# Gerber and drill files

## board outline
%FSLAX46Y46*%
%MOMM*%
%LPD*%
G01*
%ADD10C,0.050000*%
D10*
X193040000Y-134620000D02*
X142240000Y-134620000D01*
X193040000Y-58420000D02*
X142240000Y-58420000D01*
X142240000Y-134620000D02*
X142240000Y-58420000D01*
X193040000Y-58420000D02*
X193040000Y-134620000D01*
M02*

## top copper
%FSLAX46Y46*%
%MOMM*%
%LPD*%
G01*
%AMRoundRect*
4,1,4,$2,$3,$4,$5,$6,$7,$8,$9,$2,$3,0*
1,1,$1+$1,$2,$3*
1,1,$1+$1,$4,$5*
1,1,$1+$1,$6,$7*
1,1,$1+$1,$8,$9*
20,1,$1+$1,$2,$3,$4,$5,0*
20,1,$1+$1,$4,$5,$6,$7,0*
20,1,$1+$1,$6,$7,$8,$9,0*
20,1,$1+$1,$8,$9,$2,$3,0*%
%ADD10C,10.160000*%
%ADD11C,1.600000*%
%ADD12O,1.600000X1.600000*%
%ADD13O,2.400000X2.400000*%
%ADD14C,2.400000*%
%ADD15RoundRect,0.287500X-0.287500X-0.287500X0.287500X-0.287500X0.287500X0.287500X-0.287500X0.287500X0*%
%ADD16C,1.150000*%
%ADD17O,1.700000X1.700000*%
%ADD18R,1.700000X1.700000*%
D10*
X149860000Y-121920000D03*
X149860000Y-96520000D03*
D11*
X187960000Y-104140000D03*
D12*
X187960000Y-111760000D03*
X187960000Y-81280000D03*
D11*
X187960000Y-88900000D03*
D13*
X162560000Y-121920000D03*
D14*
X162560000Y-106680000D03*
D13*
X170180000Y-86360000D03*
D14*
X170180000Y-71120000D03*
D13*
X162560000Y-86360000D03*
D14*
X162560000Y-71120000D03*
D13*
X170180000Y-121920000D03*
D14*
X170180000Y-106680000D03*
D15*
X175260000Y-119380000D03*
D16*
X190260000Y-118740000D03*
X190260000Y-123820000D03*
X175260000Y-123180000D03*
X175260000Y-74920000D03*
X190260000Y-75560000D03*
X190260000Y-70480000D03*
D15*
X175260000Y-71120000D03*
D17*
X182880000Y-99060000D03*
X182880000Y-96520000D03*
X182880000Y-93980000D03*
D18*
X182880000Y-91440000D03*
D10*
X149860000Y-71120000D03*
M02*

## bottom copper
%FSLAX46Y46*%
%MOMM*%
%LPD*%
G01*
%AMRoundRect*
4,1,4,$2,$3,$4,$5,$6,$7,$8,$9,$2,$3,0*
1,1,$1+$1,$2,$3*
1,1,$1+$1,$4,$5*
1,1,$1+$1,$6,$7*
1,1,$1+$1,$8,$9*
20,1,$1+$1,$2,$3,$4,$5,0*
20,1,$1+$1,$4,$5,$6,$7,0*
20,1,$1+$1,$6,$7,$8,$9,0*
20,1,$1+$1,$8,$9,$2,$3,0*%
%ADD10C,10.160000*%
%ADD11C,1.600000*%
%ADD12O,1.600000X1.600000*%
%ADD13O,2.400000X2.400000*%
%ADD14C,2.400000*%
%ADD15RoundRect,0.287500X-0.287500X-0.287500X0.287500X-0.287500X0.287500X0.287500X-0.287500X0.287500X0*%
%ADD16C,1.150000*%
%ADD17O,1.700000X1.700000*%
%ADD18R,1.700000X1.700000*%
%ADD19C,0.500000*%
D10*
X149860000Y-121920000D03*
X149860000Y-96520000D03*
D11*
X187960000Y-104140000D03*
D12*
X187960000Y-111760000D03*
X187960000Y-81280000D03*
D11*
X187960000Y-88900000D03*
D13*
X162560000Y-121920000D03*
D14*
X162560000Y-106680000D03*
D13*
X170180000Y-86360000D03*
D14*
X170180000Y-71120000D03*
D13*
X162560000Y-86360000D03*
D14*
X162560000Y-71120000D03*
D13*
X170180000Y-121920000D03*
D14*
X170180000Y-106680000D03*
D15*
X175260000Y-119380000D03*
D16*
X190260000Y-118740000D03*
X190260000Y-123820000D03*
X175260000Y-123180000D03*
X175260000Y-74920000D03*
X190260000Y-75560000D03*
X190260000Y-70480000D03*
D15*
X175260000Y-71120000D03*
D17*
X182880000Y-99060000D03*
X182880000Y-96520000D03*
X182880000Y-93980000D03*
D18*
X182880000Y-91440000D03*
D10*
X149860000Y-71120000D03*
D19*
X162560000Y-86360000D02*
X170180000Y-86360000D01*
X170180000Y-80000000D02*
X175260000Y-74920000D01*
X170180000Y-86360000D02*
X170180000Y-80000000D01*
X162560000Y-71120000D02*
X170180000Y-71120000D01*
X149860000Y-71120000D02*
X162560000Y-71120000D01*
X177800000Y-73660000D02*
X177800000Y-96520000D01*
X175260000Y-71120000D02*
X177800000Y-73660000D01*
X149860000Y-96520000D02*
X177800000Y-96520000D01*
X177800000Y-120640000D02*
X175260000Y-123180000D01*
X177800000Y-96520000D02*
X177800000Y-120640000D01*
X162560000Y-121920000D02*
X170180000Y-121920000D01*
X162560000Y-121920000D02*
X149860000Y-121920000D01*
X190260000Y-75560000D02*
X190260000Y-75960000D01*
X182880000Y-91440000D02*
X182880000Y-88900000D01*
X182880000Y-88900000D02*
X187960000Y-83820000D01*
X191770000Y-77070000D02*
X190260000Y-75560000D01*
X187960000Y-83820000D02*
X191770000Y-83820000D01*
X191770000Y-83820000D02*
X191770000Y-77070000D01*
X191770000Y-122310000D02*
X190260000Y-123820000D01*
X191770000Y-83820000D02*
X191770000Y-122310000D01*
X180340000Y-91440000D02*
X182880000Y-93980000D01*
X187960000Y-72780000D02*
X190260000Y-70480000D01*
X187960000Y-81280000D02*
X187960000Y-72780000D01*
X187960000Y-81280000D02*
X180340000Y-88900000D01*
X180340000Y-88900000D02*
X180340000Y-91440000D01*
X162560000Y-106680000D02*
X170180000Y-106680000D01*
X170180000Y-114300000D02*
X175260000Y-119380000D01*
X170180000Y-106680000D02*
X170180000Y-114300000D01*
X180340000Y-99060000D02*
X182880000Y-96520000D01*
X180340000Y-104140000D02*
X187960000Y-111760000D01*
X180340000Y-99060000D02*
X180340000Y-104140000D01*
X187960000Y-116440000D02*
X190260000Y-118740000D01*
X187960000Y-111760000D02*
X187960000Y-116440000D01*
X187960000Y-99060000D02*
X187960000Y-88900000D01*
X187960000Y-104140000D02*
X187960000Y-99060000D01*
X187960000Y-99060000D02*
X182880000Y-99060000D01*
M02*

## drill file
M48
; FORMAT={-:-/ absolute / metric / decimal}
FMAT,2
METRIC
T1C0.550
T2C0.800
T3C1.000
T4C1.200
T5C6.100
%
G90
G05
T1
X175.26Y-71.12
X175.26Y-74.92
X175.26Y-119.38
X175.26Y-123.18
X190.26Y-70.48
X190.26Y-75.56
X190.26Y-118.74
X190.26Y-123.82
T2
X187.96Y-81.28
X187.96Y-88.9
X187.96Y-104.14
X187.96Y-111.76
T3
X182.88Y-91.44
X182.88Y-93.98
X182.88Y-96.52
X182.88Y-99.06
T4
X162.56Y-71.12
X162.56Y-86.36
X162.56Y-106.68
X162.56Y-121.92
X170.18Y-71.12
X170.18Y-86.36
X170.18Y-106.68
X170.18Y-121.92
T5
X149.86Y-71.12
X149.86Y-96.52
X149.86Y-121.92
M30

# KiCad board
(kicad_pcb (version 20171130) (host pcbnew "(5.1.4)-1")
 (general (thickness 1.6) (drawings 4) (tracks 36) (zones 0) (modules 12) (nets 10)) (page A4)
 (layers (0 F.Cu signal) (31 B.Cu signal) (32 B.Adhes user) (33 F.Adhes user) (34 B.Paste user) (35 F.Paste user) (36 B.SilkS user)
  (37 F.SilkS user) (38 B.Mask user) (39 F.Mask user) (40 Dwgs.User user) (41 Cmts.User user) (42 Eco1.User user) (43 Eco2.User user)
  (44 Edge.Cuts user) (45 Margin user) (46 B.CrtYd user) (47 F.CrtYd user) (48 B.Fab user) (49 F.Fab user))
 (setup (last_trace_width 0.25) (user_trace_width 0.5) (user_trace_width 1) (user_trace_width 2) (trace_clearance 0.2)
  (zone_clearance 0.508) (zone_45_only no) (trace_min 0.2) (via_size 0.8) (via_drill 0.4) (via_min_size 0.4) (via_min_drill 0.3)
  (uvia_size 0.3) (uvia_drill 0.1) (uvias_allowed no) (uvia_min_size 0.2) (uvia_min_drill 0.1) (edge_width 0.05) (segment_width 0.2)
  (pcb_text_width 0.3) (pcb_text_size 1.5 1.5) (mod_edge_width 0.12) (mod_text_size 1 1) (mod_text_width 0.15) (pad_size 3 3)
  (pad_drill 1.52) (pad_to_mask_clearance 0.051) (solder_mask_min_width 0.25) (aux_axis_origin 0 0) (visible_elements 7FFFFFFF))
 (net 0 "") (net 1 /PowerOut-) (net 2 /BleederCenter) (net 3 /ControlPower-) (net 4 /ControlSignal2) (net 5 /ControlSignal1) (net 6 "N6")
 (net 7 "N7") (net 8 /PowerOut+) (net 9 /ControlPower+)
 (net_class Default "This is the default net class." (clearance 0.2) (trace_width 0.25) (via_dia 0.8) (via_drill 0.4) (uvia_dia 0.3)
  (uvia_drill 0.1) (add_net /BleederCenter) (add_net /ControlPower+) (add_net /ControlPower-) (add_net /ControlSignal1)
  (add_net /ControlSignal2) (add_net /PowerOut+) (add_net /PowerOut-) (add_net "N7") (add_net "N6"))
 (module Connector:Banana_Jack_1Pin (layer F.Cu) (at 149.86 121.92)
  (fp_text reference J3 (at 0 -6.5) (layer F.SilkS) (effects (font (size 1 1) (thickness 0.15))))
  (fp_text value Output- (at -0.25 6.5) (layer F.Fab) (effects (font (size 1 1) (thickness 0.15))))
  (pad 1 thru_hole circle (at 0 0) (size 10.16 10.16) (drill 6.1) (layers *.Cu *.Mask) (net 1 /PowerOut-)))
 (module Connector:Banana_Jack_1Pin (layer F.Cu) (at 149.86 96.52)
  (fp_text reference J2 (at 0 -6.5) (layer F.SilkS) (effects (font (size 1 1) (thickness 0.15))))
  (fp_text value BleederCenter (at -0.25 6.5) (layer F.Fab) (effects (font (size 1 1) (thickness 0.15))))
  (pad 1 thru_hole circle (at 0 0) (size 10.16 10.16) (drill 6.1) (layers *.Cu *.Mask) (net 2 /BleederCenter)))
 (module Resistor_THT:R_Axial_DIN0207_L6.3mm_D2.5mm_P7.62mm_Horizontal (layer F.Cu) (at 187.96 104.14 270)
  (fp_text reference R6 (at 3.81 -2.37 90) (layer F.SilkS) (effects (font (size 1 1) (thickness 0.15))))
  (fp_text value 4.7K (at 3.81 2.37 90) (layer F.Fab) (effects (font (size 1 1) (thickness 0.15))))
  (pad 1 thru_hole circle (at 0 0 270) (size 1.6 1.6) (drill 0.8) (layers *.Cu *.Mask) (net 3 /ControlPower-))
  (pad 2 thru_hole oval (at 7.62 0 270) (size 1.6 1.6) (drill 0.8) (layers *.Cu *.Mask) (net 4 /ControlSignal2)))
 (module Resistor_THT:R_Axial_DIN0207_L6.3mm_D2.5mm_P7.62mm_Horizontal (layer F.Cu) (at 187.96 88.9 90)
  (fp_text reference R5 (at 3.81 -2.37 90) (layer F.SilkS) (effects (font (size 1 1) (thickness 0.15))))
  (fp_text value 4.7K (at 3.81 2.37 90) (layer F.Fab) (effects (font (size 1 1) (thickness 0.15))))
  (pad 2 thru_hole oval (at 7.62 0 90) (size 1.6 1.6) (drill 0.8) (layers *.Cu *.Mask) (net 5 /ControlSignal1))
  (pad 1 thru_hole circle (at 0 0 90) (size 1.6 1.6) (drill 0.8) (layers *.Cu *.Mask) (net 3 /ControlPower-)))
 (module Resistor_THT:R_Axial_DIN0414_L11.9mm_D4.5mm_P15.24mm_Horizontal (layer F.Cu) (at 162.56 106.68 270)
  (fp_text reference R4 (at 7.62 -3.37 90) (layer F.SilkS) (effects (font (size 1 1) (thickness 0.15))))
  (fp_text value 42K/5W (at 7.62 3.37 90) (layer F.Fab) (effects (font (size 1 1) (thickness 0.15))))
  (pad 2 thru_hole oval (at 15.24 0 270) (size 2.4 2.4) (drill 1.2) (layers *.Cu *.Mask) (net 1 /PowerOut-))
  (pad 1 thru_hole circle (at 0 0 270) (size 2.4 2.4) (drill 1.2) (layers *.Cu *.Mask) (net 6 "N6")))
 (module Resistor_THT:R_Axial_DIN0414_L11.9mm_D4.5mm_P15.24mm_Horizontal (layer F.Cu) (at 170.18 71.12 270)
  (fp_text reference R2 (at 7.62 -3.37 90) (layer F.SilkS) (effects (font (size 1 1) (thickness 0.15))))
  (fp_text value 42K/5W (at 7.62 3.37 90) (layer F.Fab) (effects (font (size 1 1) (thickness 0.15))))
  (pad 2 thru_hole oval (at 15.24 0 270) (size 2.4 2.4) (drill 1.2) (layers *.Cu *.Mask) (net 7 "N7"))
  (pad 1 thru_hole circle (at 0 0 270) (size 2.4 2.4) (drill 1.2) (layers *.Cu *.Mask) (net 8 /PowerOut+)))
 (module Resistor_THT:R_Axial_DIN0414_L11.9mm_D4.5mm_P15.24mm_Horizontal (layer F.Cu) (at 162.56 71.12 270)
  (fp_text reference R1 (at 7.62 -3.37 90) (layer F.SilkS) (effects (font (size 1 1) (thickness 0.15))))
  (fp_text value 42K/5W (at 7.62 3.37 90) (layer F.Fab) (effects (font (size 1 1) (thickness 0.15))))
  (pad 2 thru_hole oval (at 15.24 0 270) (size 2.4 2.4) (drill 1.2) (layers *.Cu *.Mask) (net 7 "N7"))
  (pad 1 thru_hole circle (at 0 0 270) (size 2.4 2.4) (drill 1.2) (layers *.Cu *.Mask) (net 8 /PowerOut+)))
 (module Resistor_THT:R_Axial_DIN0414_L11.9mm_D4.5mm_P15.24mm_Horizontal (layer F.Cu) (at 170.18 106.68 270)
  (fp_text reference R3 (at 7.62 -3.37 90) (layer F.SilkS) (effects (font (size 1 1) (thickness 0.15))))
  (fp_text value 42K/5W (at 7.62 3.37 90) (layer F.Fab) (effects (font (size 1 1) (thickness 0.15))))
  (pad 2 thru_hole oval (at 15.24 0 270) (size 2.4 2.4) (drill 1.2) (layers *.Cu *.Mask) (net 1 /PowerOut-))
  (pad 1 thru_hole circle (at 0 0 270) (size 2.4 2.4) (drill 1.2) (layers *.Cu *.Mask) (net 6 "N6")))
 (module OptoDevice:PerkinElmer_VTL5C (layer F.Cu) (at 175.26 119.38)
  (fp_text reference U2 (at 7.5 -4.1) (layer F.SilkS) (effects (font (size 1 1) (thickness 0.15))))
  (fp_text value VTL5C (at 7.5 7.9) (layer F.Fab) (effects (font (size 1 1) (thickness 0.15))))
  (pad 1 thru_hole roundrect (at 0 0) (size 1.15 1.15) (drill 0.55) (layers *.Cu *.Mask) (roundrect_rratio 0.25) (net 6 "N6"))
  (pad 3 thru_hole circle (at 15 -0.64) (size 1.15 1.15) (drill 0.55) (layers *.Cu *.Mask) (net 4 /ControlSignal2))
  (pad 4 thru_hole circle (at 15 4.44) (size 1.15 1.15) (drill 0.55) (layers *.Cu *.Mask) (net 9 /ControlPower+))
  (pad 2 thru_hole circle (at 0 3.8) (size 1.15 1.15) (drill 0.55) (layers *.Cu *.Mask) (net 2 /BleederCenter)))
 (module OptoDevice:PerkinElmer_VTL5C (layer F.Cu) (at 175.26 71.12)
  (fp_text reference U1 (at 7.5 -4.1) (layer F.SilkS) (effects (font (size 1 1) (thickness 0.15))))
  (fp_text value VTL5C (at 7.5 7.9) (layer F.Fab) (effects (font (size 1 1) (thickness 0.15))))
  (pad 2 thru_hole circle (at 0 3.8) (size 1.15 1.15) (drill 0.55) (layers *.Cu *.Mask) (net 7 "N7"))
  (pad 4 thru_hole circle (at 15 4.44) (size 1.15 1.15) (drill 0.55) (layers *.Cu *.Mask) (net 9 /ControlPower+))
  (pad 3 thru_hole circle (at 15 -0.64) (size 1.15 1.15) (drill 0.55) (layers *.Cu *.Mask) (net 5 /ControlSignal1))
  (pad 1 thru_hole roundrect (at 0 0) (size 1.15 1.15) (drill 0.55) (layers *.Cu *.Mask) (roundrect_rratio 0.25) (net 2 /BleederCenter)))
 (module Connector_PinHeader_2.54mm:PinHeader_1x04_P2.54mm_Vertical (layer F.Cu) (at 182.88 91.44)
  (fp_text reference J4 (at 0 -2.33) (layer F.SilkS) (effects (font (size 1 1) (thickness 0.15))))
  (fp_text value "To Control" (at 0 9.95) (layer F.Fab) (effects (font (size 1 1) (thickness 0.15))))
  (pad 4 thru_hole oval (at 0 7.62) (size 1.7 1.7) (drill 1) (layers *.Cu *.Mask) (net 3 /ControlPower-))
  (pad 3 thru_hole oval (at 0 5.08) (size 1.7 1.7) (drill 1) (layers *.Cu *.Mask) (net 4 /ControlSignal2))
  (pad 2 thru_hole oval (at 0 2.54) (size 1.7 1.7) (drill 1) (layers *.Cu *.Mask) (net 5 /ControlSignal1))
  (pad 1 thru_hole rect (at 0 0) (size 1.7 1.7) (drill 1) (layers *.Cu *.Mask) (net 9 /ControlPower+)))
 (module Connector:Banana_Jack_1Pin (layer F.Cu) (at 149.86 71.12)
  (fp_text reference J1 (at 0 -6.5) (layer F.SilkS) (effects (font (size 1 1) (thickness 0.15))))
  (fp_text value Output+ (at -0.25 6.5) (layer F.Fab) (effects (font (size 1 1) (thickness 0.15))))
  (pad 1 thru_hole circle (at 0 0) (size 10.16 10.16) (drill 6.1) (layers *.Cu *.Mask) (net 8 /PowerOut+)))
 (gr_line (start 193.04 134.62) (end 142.24 134.62) (layer Edge.Cuts) (width 0.05))
 (gr_line (start 193.04 58.42) (end 142.24 58.42) (layer Edge.Cuts) (width 0.05))
 (gr_line (start 142.24 134.62) (end 142.24 58.42) (layer Edge.Cuts) (width 0.05))
 (gr_line (start 193.04 58.42) (end 193.04 134.62) (layer Edge.Cuts) (width 0.05))
 (segment (start 162.56 86.36) (end 170.18 86.36) (width 0.5) (layer B.Cu) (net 7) (status 30))
 (segment (start 170.18 80) (end 175.26 74.92) (width 0.5) (layer B.Cu) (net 7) (status 20))
 (segment (start 170.18 86.36) (end 170.18 80) (width 0.5) (layer B.Cu) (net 7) (status 10))
 (segment (start 162.56 71.12) (end 170.18 71.12) (width 0.5) (layer B.Cu) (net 8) (status 30))
 (segment (start 149.86 71.12) (end 162.56 71.12) (width 0.5) (layer B.Cu) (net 8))
 (segment (start 177.8 73.66) (end 177.8 96.52) (width 0.5) (layer B.Cu) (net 2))
 (segment (start 175.26 71.12) (end 177.8 73.66) (width 0.5) (layer B.Cu) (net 2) (status 10))
 (segment (start 149.86 96.52) (end 177.8 96.52) (width 0.5) (layer B.Cu) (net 2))
 (segment (start 177.8 120.64) (end 175.26 123.18) (width 0.5) (layer B.Cu) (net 2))
 (segment (start 177.8 96.52) (end 177.8 120.64) (width 0.5) (layer B.Cu) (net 2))
 (segment (start 162.56 121.92) (end 170.18 121.92) (width 0.5) (layer B.Cu) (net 1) (status 30))
 (segment (start 162.56 121.92) (end 149.86 121.92) (width 0.5) (layer B.Cu) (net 1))
 (segment (start 190.26 75.56) (end 190.26 75.96) (width 0.5) (layer B.Cu) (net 9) (status 30))
 (segment (start 182.88 91.44) (end 182.88 88.9) (width 0.5) (layer B.Cu) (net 9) (status 10))
 (segment (start 182.88 88.9) (end 187.96 83.82) (width 0.5) (layer B.Cu) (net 9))
 (segment (start 191.77 77.07) (end 190.26 75.56) (width 0.5) (layer B.Cu) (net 9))
 (segment (start 187.96 83.82) (end 191.77 83.82) (width 0.5) (layer B.Cu) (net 9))
 (segment (start 191.77 83.82) (end 191.77 77.07) (width 0.5) (layer B.Cu) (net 9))
 (segment (start 191.77 122.31) (end 190.26 123.82) (width 0.5) (layer B.Cu) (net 9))
 (segment (start 191.77 83.82) (end 191.77 122.31) (width 0.5) (layer B.Cu) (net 9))
 (segment (start 180.34 91.44) (end 182.88 93.98) (width 0.5) (layer B.Cu) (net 5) (status 20))
 (segment (start 187.96 72.78) (end 190.26 70.48) (width 0.5) (layer B.Cu) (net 5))
 (segment (start 187.96 81.28) (end 187.96 72.78) (width 0.5) (layer B.Cu) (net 5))
 (segment (start 187.96 81.28) (end 180.34 88.9) (width 0.5) (layer B.Cu) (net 5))
 (segment (start 180.34 88.9) (end 180.34 91.44) (width 0.5) (layer B.Cu) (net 5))
 (segment (start 162.56 106.68) (end 170.18 106.68) (width 0.5) (layer B.Cu) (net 6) (status 30))
 (segment (start 170.18 114.3) (end 175.26 119.38) (width 0.5) (layer B.Cu) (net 6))
 (segment (start 170.18 106.68) (end 170.18 114.3) (width 0.5) (layer B.Cu) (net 6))
 (segment (start 180.34 99.06) (end 182.88 96.52) (width 0.5) (layer B.Cu) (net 4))
 (segment (start 180.34 104.14) (end 187.96 111.76) (width 0.5) (layer B.Cu) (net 4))
 (segment (start 180.34 99.06) (end 180.34 104.14) (width 0.5) (layer B.Cu) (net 4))
 (segment (start 187.96 116.44) (end 190.26 118.74) (width 0.5) (layer B.Cu) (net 4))
 (segment (start 187.96 111.76) (end 187.96 116.44) (width 0.5) (layer B.Cu) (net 4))
 (segment (start 187.96 99.06) (end 187.96 88.9) (width 0.5) (layer B.Cu) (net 3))
 (segment (start 187.96 104.14) (end 187.96 99.06) (width 0.5) (layer B.Cu) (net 3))
 (segment (start 187.96 99.06) (end 182.88 99.06) (width 0.5) (layer B.Cu) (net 3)))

